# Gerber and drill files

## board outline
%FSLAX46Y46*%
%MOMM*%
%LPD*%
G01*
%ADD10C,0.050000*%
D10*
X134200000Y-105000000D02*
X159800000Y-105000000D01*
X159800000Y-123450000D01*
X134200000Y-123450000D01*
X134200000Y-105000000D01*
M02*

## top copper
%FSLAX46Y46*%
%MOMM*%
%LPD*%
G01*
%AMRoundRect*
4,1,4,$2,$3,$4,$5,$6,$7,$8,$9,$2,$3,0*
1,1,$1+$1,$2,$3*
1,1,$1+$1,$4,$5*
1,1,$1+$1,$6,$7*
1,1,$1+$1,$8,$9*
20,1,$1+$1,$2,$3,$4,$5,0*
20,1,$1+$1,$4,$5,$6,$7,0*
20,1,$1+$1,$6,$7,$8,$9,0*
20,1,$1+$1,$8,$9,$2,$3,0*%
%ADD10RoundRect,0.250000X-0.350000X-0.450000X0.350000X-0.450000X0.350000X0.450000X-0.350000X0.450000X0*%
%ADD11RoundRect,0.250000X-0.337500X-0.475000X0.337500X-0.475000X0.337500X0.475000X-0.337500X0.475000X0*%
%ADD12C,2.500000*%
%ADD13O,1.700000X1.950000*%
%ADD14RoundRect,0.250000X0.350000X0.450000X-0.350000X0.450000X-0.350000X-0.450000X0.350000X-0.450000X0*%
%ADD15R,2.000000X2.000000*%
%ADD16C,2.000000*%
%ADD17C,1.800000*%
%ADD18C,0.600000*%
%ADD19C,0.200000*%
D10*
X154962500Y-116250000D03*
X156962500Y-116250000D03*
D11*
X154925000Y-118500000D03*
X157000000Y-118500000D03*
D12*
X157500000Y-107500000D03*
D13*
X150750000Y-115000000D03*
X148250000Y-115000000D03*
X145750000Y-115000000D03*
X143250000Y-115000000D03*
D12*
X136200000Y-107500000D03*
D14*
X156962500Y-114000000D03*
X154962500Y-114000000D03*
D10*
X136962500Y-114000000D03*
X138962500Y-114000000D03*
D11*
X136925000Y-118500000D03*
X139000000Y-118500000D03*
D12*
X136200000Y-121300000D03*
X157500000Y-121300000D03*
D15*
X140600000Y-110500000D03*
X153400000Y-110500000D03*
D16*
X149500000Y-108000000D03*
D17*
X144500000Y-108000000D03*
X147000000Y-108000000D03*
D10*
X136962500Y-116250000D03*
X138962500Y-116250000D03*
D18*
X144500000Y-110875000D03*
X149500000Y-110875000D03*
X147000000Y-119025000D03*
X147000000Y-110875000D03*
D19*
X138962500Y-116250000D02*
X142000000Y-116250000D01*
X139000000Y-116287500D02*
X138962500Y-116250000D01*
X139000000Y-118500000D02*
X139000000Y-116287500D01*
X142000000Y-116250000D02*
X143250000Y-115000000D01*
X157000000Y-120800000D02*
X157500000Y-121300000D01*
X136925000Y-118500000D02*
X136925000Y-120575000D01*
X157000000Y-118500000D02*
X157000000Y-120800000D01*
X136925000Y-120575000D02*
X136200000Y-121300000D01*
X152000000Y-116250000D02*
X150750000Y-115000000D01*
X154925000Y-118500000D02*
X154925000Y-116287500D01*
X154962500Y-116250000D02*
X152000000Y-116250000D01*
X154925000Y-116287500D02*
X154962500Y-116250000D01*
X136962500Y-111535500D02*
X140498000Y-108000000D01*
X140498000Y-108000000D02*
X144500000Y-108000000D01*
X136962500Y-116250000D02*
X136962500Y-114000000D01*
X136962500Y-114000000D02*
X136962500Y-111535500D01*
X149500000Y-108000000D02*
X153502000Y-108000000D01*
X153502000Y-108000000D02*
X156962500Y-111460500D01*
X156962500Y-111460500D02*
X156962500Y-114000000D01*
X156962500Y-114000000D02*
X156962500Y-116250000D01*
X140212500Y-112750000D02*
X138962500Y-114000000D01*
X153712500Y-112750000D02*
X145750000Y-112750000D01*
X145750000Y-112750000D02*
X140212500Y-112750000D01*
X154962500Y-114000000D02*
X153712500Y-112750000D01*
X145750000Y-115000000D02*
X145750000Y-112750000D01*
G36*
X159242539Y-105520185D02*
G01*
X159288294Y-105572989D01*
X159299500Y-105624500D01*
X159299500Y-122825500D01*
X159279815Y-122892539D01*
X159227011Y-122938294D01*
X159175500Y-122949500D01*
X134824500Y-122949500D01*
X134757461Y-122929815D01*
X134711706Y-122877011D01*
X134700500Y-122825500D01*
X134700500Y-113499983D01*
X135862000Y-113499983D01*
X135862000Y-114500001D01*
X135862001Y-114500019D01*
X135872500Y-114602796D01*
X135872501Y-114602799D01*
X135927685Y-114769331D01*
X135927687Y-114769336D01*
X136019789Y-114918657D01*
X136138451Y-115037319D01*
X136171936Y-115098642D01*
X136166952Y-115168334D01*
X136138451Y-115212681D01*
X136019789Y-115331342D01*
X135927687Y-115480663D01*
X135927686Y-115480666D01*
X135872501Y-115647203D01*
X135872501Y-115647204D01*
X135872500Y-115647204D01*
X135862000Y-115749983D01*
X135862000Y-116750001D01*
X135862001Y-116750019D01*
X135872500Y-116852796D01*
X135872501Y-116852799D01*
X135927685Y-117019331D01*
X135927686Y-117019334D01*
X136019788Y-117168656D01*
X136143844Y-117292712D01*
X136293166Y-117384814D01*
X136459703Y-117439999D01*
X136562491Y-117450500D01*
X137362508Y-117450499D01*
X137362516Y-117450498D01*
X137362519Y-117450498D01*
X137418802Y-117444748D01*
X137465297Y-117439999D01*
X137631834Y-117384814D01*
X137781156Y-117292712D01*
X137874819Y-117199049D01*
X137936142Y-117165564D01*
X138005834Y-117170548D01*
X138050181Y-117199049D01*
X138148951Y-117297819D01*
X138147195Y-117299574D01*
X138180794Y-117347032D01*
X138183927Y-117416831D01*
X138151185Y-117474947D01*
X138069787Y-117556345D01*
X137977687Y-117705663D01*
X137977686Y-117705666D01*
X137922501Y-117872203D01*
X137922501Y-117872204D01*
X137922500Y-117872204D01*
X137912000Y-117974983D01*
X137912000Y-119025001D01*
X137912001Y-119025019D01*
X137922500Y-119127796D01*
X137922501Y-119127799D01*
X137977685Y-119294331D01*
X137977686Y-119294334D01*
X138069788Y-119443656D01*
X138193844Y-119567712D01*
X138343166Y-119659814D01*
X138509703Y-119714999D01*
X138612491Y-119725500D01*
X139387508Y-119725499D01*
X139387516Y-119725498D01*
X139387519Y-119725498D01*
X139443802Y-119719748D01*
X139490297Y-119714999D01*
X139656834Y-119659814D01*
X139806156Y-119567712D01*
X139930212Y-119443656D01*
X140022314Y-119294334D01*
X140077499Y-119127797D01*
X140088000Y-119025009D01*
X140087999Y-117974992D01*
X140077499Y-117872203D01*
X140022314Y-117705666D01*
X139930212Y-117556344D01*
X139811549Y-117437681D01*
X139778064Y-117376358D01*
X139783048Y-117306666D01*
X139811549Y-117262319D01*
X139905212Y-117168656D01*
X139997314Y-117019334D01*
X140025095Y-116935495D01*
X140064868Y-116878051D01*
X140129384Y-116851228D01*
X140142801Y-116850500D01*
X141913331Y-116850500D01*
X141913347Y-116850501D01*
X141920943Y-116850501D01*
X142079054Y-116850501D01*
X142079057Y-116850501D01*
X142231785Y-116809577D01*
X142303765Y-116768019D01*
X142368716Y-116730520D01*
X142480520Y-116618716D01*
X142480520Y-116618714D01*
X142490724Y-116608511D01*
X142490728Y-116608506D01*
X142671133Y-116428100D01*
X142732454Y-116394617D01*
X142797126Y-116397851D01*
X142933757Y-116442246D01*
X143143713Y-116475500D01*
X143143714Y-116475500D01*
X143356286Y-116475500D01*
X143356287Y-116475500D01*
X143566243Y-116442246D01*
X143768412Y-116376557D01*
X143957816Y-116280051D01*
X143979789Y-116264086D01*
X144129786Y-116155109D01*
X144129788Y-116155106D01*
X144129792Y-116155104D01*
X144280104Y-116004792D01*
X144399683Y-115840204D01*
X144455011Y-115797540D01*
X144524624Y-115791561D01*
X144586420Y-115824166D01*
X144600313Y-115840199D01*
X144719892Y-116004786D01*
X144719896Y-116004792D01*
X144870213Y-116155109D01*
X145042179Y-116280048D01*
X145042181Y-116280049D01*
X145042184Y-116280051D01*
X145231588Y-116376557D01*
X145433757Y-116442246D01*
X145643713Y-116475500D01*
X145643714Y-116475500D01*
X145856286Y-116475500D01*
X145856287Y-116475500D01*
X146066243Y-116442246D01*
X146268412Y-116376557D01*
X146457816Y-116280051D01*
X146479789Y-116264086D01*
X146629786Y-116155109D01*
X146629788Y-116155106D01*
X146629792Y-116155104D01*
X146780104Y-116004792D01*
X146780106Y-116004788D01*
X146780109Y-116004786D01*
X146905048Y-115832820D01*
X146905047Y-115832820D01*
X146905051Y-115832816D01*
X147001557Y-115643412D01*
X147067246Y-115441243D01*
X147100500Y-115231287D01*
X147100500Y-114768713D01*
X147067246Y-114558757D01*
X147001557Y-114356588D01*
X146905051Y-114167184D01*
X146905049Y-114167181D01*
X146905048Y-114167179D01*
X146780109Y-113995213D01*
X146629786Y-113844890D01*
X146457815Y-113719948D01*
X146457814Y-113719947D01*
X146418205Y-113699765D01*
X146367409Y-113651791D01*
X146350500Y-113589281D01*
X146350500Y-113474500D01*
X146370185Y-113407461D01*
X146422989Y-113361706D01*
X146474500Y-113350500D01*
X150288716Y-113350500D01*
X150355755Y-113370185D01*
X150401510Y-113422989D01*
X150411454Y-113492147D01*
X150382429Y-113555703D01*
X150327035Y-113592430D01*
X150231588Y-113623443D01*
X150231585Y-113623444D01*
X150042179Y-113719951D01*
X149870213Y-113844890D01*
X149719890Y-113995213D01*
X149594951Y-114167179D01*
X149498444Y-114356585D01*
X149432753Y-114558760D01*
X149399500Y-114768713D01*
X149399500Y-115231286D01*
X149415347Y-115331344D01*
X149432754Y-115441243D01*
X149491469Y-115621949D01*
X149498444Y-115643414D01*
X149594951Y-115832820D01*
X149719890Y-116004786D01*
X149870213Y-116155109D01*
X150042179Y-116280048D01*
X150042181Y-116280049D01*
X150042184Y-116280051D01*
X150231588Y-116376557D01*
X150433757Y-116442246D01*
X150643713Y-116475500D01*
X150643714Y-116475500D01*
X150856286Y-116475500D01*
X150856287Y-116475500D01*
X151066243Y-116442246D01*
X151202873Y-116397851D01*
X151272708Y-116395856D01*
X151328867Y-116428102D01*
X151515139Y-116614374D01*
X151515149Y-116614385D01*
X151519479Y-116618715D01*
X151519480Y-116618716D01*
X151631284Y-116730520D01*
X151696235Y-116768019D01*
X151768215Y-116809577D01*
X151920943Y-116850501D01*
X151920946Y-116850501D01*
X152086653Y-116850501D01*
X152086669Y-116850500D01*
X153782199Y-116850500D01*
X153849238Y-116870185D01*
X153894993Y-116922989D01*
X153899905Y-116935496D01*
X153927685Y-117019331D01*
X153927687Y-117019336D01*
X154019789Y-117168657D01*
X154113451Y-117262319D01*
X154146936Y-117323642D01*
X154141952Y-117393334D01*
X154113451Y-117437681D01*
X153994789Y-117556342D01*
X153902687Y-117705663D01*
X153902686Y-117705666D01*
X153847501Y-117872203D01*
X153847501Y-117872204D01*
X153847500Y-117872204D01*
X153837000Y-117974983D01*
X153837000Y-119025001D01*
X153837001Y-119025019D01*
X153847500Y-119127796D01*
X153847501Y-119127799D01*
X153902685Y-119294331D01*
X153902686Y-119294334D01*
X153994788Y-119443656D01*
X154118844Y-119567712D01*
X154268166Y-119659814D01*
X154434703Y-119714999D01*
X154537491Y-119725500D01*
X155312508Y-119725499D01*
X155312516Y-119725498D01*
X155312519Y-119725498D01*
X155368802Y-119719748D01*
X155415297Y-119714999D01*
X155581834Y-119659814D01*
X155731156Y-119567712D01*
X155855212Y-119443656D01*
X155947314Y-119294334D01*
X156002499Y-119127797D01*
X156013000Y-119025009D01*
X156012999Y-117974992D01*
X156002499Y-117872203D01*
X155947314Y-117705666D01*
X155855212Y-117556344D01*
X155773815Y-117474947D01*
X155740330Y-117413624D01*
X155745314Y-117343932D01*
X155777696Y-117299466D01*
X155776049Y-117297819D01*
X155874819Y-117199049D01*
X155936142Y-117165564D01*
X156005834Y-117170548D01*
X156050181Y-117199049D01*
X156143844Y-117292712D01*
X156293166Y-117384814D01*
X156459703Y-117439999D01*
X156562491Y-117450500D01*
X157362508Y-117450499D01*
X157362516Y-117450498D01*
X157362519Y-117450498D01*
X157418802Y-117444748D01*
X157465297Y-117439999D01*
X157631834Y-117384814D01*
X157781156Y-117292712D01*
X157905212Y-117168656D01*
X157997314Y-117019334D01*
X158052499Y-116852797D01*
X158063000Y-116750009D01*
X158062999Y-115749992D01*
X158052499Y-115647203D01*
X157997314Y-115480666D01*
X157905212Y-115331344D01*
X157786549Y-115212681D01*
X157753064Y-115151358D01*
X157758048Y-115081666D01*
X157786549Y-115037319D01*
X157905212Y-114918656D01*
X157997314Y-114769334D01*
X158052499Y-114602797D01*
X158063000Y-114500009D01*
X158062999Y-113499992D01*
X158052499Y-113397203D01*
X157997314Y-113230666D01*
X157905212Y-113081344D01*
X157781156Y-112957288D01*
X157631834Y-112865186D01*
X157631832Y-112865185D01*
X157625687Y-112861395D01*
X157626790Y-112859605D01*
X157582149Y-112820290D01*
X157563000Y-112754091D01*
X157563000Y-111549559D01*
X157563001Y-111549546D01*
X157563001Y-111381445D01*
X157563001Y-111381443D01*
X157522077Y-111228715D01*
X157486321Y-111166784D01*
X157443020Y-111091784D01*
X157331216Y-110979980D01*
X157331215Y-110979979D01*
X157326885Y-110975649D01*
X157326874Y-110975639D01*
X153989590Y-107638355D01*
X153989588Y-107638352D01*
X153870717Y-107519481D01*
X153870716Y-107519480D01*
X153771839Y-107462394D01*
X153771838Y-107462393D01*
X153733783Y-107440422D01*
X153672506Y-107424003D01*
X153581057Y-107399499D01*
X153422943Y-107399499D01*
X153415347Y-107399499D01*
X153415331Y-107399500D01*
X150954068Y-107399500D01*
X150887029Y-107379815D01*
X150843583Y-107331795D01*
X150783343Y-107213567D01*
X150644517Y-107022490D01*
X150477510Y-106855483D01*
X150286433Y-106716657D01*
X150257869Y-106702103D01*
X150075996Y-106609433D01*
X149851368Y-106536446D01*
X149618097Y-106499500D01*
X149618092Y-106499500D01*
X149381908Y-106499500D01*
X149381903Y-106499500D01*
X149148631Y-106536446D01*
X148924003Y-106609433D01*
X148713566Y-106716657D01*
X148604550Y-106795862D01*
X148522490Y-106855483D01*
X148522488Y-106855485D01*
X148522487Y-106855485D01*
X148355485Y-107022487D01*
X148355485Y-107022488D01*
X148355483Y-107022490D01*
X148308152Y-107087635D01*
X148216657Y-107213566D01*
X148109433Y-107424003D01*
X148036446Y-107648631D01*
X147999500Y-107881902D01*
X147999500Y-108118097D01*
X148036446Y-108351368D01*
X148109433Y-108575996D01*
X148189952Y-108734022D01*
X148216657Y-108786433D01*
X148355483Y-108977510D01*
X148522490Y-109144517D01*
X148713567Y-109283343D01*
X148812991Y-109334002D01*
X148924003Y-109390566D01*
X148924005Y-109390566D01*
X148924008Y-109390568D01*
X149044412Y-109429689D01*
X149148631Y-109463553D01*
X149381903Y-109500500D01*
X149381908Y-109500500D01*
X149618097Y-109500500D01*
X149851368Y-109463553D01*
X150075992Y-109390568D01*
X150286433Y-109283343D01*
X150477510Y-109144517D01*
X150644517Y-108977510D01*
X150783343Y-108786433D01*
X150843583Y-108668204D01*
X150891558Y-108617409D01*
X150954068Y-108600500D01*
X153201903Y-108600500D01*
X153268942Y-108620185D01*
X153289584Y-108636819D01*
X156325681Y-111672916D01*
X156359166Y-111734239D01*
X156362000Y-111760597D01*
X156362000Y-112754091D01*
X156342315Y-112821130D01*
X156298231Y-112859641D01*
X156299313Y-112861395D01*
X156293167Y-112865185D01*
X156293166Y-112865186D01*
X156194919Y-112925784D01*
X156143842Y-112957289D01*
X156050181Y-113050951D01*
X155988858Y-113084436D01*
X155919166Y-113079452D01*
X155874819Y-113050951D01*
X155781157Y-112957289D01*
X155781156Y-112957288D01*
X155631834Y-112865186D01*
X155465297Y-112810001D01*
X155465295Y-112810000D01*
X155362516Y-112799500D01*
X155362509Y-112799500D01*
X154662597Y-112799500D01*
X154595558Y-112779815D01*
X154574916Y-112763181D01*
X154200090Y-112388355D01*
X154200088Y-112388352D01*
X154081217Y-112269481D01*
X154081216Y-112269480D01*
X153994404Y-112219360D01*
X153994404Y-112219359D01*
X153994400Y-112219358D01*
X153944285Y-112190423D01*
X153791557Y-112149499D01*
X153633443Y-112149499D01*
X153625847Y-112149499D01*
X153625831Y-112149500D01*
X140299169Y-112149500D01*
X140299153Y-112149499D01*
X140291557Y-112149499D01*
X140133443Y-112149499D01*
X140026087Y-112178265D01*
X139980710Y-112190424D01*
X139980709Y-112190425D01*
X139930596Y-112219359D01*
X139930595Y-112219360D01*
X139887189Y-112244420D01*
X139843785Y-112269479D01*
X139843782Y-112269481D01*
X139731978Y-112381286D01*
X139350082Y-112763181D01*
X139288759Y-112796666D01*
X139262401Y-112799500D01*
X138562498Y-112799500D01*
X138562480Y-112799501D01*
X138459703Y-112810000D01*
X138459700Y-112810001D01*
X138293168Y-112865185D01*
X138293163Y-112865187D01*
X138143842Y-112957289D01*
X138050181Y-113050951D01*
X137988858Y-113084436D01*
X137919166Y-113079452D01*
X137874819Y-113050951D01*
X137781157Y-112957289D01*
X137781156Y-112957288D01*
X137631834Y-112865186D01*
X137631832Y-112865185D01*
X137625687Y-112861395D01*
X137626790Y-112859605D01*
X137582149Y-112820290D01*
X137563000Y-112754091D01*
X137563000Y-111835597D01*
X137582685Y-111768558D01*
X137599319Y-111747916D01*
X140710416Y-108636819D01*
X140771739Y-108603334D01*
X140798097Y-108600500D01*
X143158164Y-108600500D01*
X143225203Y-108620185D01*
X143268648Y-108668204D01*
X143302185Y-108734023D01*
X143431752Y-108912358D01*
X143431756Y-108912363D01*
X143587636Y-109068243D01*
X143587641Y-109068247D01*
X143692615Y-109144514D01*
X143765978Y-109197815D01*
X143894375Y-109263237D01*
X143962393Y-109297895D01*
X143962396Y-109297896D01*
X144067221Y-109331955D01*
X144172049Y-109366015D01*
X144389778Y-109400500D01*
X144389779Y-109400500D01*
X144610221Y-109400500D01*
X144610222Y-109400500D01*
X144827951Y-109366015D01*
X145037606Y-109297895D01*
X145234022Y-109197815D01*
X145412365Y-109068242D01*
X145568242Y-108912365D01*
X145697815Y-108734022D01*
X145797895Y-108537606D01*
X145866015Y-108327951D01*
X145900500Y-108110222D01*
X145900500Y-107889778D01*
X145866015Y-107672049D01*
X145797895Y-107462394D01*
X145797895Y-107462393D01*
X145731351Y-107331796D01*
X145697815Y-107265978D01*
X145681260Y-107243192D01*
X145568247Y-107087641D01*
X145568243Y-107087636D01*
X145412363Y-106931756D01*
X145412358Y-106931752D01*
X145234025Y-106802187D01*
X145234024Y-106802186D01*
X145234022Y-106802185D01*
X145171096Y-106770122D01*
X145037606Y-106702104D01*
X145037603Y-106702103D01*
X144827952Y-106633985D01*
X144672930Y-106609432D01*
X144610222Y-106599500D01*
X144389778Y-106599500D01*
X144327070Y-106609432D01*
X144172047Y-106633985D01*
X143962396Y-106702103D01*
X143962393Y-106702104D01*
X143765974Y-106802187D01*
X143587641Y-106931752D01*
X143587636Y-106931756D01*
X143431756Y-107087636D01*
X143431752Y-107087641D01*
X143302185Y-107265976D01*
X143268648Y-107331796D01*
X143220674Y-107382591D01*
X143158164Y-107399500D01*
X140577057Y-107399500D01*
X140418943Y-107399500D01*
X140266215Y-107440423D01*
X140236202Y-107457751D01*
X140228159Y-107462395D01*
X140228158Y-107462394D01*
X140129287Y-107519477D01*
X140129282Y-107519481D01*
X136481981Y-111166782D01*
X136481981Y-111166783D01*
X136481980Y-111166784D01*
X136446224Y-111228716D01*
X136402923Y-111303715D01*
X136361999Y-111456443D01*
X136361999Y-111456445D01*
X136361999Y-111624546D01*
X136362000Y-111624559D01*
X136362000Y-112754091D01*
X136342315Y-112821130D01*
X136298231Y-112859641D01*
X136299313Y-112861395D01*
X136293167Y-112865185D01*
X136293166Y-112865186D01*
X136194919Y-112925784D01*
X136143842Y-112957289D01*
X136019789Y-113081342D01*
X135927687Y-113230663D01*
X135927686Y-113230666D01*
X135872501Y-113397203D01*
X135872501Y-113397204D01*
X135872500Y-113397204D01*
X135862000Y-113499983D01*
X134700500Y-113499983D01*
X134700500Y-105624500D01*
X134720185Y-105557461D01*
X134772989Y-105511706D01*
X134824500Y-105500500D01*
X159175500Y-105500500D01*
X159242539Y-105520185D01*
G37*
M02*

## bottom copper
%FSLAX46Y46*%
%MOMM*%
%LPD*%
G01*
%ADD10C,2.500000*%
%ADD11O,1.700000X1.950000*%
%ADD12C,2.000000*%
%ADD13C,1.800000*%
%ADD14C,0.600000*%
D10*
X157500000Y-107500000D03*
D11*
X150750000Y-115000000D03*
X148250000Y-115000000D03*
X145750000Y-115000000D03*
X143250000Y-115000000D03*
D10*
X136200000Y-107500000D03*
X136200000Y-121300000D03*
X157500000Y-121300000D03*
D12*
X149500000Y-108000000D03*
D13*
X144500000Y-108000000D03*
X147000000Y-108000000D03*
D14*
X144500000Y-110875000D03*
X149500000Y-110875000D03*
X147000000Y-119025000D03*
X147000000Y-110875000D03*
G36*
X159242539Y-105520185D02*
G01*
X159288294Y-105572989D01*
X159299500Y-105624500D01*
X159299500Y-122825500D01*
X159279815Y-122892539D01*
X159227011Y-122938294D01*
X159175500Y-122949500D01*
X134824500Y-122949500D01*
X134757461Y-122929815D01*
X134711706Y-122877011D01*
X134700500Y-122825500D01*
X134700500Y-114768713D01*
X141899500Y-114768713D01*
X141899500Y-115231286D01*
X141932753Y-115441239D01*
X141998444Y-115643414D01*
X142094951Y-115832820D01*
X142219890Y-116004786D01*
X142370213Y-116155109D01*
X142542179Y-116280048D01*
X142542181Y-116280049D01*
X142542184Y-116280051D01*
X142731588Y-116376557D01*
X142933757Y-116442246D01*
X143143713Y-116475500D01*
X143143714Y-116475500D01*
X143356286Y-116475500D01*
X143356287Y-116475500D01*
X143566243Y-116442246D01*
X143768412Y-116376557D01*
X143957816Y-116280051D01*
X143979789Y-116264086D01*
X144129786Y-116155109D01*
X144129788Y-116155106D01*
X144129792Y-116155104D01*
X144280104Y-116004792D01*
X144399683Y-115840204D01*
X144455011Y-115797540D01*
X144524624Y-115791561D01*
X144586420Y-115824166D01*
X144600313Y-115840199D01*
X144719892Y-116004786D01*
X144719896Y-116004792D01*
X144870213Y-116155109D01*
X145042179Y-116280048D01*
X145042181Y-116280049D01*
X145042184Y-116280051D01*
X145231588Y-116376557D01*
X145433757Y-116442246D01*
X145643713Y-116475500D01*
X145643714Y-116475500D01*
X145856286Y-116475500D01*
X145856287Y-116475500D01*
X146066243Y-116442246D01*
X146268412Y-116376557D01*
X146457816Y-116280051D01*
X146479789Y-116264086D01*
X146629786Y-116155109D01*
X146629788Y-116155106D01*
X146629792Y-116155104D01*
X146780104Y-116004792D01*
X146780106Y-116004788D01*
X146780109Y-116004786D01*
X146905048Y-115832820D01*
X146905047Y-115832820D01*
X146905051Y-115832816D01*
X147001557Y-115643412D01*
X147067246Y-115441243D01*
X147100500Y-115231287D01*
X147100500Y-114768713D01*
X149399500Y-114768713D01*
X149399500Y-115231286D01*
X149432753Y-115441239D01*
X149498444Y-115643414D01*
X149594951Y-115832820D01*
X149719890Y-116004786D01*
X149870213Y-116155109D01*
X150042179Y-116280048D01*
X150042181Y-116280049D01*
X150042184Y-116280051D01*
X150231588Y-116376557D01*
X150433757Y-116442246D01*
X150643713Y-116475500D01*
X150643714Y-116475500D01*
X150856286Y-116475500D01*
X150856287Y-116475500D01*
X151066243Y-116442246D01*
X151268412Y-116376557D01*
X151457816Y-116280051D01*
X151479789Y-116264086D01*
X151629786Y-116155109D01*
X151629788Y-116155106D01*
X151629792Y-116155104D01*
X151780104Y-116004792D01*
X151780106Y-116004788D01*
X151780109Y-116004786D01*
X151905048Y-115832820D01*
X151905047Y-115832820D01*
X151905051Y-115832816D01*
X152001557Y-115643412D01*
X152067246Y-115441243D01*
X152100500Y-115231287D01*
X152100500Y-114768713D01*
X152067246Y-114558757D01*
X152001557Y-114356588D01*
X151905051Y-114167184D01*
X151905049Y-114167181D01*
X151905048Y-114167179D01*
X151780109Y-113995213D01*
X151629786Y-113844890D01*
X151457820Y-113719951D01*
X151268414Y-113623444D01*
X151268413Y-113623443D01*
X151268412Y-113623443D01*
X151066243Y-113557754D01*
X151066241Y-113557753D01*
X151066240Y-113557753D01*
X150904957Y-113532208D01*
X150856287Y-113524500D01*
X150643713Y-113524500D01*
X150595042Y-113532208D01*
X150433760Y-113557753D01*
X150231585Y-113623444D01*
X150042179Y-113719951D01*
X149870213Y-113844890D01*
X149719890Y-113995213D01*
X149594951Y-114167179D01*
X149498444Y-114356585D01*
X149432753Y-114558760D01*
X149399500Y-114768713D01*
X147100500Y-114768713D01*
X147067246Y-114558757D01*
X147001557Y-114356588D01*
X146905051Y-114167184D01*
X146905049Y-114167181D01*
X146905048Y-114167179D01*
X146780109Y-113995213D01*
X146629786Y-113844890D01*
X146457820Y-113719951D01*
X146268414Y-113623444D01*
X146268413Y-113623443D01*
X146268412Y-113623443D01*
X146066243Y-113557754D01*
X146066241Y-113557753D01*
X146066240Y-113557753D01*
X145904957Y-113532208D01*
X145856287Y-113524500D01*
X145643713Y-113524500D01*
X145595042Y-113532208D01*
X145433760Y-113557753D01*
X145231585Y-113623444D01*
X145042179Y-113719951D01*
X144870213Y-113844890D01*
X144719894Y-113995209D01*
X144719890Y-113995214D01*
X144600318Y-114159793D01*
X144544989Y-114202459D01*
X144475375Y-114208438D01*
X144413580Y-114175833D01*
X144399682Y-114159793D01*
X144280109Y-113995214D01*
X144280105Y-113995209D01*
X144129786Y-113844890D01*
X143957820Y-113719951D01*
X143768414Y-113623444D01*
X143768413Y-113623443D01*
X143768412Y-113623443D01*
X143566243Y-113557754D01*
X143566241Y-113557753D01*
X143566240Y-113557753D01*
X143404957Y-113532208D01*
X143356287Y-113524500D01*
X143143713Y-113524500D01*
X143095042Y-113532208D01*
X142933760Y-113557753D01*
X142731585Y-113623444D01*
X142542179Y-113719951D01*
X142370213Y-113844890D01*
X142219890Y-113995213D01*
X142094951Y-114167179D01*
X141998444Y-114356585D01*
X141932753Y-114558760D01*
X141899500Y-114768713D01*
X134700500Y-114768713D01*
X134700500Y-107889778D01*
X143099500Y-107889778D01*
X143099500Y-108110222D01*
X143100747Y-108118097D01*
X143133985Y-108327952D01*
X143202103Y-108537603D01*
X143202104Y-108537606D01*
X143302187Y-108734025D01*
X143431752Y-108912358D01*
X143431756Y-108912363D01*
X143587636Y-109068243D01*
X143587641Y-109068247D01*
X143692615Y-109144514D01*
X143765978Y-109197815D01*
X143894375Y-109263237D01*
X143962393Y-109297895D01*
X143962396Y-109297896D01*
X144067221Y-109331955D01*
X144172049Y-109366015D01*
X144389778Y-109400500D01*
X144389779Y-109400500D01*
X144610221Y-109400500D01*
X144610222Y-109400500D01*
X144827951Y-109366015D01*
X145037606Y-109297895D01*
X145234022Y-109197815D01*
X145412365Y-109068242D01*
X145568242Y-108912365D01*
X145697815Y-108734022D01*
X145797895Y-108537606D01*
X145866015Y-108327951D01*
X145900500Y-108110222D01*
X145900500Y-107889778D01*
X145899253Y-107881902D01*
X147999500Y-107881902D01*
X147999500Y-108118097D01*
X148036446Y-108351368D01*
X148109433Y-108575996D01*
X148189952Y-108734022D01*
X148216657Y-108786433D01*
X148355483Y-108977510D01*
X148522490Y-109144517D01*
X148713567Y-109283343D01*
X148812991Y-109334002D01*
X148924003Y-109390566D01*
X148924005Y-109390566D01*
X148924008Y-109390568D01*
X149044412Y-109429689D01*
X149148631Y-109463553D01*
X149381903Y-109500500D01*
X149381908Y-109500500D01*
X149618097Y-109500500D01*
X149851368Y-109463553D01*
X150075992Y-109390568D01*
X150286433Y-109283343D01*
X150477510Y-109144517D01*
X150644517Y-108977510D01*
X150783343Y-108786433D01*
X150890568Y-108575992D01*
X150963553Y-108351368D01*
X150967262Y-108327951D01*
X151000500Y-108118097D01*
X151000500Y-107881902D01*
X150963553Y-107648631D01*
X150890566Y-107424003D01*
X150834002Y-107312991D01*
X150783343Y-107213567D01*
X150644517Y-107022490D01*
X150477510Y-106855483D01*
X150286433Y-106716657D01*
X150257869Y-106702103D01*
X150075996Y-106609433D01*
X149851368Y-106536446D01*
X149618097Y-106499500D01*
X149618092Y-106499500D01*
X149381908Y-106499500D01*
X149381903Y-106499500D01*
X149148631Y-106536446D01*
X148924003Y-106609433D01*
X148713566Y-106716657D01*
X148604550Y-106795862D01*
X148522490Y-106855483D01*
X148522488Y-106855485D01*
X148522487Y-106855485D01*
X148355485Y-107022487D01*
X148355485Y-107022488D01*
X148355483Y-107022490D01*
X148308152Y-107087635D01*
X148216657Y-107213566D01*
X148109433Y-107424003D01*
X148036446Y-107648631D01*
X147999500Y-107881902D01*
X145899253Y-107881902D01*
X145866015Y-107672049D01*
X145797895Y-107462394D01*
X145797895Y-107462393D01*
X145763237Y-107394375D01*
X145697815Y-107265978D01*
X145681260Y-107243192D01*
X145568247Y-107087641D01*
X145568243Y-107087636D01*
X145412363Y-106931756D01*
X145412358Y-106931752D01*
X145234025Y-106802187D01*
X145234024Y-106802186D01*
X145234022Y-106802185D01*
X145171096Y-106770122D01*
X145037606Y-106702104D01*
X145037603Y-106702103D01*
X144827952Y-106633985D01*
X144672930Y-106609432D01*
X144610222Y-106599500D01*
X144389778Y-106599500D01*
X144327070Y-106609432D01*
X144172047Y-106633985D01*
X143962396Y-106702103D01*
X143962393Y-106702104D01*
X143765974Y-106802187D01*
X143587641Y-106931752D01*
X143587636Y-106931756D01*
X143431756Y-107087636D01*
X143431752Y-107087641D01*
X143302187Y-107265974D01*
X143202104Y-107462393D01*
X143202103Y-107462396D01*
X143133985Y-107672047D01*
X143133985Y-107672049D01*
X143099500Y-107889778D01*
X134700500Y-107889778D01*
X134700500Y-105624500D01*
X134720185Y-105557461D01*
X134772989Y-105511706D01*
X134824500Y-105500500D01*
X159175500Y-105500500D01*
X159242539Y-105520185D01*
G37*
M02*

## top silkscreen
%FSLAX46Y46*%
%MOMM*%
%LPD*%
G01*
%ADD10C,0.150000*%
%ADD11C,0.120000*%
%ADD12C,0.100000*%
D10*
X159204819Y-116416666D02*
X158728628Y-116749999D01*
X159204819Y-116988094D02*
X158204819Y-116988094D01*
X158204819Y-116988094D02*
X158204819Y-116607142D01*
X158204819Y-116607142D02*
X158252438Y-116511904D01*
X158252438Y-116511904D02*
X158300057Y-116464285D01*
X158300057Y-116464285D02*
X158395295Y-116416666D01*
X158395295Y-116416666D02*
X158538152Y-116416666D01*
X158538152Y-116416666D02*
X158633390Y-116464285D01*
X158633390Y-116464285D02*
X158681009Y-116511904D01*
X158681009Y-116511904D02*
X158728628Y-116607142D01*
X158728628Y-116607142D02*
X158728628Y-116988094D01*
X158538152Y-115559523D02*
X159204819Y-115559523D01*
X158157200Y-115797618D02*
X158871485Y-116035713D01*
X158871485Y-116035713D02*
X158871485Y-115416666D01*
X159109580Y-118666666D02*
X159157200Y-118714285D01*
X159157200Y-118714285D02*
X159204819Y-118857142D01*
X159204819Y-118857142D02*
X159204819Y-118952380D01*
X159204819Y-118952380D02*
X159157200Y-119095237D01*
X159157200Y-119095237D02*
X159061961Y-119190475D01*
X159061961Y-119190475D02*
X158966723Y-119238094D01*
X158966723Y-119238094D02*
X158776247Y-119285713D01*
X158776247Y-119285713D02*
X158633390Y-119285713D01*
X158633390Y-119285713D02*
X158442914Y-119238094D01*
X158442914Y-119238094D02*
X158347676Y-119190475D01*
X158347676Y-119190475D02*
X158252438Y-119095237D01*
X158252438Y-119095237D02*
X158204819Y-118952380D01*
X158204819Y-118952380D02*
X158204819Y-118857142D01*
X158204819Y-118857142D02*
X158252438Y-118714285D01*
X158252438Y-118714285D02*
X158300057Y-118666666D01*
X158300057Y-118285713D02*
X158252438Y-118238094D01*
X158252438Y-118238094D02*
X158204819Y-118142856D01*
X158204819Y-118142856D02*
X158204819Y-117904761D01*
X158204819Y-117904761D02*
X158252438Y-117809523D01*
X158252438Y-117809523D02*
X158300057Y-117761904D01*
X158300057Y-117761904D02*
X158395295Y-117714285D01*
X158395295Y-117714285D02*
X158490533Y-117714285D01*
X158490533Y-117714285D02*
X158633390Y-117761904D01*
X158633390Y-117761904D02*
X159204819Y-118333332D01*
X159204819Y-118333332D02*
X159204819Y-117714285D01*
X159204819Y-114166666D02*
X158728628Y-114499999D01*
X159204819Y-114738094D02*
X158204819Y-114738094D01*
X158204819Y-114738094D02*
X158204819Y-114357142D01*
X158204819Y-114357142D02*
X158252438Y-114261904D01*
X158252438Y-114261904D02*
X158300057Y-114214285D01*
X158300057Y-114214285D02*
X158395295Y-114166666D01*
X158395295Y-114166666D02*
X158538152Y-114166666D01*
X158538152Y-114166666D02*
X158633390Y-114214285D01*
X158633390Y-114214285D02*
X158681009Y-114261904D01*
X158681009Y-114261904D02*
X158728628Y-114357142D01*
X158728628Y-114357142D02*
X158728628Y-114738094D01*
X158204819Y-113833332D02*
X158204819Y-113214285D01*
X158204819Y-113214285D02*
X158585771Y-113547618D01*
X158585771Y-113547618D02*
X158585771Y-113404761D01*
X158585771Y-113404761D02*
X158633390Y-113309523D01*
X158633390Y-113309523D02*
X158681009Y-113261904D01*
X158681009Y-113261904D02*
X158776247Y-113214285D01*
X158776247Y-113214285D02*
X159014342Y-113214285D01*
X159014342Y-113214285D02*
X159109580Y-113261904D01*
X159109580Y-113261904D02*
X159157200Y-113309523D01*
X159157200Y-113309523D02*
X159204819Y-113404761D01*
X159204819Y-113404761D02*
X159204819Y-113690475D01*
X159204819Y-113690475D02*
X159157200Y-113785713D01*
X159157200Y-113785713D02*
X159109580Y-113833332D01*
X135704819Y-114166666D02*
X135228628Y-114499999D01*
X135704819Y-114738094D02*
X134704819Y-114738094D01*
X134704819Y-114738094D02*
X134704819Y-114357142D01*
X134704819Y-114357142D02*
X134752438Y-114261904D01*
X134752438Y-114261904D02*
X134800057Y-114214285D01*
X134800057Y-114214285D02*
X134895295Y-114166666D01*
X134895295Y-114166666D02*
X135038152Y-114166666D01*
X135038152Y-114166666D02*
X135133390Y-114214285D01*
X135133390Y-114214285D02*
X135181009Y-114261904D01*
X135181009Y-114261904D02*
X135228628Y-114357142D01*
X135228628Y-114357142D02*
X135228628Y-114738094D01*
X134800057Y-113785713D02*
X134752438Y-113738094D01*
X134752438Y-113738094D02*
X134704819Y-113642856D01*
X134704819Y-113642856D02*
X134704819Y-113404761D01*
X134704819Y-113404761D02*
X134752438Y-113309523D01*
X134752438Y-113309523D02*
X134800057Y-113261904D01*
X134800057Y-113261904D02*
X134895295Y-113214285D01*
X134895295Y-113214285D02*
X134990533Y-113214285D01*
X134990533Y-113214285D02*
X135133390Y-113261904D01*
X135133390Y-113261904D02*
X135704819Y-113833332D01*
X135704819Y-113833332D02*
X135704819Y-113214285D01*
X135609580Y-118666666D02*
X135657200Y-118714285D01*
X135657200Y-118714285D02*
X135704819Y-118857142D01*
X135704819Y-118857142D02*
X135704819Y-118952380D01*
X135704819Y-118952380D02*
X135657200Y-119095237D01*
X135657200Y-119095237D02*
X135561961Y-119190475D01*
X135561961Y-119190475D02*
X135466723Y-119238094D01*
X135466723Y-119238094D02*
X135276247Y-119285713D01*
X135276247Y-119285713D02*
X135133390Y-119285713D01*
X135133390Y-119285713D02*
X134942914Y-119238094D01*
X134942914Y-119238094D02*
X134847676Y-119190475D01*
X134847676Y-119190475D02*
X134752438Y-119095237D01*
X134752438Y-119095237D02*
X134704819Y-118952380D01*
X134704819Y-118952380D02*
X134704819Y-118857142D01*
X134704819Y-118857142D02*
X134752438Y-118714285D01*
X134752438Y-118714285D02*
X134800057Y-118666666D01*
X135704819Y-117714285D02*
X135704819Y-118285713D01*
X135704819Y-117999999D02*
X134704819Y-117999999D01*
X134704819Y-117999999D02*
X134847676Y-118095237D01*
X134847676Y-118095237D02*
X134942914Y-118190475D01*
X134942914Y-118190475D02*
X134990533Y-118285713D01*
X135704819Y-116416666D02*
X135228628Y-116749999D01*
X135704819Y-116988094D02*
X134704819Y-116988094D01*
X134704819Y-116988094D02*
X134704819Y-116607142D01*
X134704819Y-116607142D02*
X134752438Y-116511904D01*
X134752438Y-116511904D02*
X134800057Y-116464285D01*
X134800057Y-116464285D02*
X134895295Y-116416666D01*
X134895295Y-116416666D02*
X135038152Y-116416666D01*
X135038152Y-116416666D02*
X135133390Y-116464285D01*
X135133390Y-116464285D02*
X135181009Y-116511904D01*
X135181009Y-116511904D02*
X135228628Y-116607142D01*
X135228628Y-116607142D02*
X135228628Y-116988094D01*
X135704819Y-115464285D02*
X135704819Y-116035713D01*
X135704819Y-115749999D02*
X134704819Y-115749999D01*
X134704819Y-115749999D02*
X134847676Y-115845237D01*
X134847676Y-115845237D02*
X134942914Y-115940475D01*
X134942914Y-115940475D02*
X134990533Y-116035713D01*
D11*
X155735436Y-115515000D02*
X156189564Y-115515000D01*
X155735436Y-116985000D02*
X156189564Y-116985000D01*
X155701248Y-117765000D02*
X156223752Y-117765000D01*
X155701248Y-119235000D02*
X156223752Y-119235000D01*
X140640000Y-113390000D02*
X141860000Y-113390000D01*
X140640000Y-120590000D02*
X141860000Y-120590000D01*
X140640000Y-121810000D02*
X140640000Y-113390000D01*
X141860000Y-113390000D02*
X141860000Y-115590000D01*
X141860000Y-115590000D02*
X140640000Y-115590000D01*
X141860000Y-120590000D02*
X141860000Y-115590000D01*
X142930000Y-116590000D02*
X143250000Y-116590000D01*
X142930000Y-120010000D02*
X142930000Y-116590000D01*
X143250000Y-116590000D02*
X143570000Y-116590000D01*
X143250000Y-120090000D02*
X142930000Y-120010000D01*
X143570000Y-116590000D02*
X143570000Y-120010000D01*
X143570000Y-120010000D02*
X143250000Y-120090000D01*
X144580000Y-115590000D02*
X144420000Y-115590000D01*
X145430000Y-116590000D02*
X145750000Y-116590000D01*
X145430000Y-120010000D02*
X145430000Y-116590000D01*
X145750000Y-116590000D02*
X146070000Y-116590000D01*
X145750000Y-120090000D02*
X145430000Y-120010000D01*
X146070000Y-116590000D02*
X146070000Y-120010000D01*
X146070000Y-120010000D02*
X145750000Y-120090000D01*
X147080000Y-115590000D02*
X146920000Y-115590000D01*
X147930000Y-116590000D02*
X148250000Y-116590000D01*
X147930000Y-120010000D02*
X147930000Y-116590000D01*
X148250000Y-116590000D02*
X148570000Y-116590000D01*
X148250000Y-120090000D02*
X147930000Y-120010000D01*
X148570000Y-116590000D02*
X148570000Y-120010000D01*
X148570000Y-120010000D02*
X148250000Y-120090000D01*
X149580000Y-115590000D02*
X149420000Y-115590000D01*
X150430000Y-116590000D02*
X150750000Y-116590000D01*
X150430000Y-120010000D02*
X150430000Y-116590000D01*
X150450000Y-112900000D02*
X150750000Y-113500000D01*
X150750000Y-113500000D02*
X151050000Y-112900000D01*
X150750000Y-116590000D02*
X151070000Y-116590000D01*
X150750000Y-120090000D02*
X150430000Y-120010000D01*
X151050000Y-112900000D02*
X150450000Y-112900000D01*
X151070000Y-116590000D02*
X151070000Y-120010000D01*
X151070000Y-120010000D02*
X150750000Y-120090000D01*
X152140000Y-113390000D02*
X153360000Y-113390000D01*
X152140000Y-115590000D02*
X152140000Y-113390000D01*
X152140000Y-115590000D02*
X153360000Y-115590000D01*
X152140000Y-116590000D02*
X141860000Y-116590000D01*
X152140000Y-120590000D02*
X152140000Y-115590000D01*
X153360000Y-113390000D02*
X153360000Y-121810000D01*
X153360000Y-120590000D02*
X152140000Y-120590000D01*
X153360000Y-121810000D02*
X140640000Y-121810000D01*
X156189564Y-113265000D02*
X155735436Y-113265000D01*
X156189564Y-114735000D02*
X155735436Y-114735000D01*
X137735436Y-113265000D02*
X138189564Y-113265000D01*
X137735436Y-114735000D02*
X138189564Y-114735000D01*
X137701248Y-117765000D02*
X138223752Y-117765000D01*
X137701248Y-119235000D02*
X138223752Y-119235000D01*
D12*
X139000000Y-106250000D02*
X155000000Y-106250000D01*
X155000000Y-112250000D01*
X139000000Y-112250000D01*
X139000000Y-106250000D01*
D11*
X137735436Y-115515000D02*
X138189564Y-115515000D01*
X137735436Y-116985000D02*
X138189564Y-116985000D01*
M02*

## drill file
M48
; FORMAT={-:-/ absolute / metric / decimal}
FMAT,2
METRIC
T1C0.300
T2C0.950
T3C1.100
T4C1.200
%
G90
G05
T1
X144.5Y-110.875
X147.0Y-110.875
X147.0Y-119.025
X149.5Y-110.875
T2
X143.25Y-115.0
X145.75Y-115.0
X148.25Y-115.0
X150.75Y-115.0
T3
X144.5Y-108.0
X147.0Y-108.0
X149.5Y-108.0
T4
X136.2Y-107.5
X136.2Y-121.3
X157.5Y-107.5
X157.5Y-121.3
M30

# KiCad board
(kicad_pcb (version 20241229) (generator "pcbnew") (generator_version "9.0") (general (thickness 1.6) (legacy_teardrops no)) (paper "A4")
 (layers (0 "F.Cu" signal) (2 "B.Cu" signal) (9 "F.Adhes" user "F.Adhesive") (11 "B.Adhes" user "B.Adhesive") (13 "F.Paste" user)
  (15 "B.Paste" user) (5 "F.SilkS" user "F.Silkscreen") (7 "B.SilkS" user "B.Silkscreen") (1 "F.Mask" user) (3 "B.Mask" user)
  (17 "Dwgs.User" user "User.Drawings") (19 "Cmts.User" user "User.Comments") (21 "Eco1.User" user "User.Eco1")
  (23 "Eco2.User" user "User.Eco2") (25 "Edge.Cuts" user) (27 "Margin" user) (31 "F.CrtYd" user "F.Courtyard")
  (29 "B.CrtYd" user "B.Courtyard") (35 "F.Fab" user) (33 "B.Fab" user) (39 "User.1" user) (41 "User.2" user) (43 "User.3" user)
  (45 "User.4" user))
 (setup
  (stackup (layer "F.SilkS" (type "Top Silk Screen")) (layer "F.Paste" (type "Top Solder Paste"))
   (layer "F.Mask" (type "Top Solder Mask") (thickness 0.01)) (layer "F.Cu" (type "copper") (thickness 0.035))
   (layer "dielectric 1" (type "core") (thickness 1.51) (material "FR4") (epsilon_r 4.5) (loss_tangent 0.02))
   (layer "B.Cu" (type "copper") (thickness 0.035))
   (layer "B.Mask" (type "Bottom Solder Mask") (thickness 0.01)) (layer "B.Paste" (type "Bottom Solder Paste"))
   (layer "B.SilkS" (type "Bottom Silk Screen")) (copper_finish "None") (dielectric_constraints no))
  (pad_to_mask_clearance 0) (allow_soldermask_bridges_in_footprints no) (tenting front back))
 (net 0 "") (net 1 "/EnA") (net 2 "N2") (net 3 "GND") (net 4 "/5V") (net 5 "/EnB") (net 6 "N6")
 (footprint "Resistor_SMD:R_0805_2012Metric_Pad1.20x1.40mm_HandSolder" (layer "F.Cu") (at 155.9625 116.25)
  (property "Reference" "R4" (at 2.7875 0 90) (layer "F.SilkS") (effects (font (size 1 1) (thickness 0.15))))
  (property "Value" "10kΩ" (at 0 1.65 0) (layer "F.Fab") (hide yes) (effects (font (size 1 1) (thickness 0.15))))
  (fp_line (start -0.227064 -0.735) (end 0.227064 -0.735) (stroke (width 0.12) (type solid)) (layer "F.SilkS"))
  (fp_line (start -0.227064 0.735) (end 0.227064 0.735) (stroke (width 0.12) (type solid)) (layer "F.SilkS"))
  (pad "1" smd roundrect (at -1 0) (size 1.2 1.4) (layers "F.Cu" "F.Mask" "F.Paste") (roundrect_rratio 0.208333) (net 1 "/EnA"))
  (pad "2" smd roundrect (at 1 0) (size 1.2 1.4) (layers "F.Cu" "F.Mask" "F.Paste") (roundrect_rratio 0.208333) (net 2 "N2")))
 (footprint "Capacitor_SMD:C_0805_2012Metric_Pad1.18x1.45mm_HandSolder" (layer "F.Cu") (at 155.9625 118.5)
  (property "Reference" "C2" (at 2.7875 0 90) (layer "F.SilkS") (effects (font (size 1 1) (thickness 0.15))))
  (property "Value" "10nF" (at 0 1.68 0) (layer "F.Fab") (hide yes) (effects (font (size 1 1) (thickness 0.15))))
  (fp_line (start -0.261252 -0.735) (end 0.261252 -0.735) (stroke (width 0.12) (type solid)) (layer "F.SilkS"))
  (fp_line (start -0.261252 0.735) (end 0.261252 0.735) (stroke (width 0.12) (type solid)) (layer "F.SilkS"))
  (pad "1" smd roundrect (at -1.0375 0) (size 1.175 1.45) (layers "F.Cu" "F.Mask" "F.Paste") (roundrect_rratio 0.212766) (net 1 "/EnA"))
  (pad "2" smd roundrect (at 1.0375 0) (size 1.175 1.45) (layers "F.Cu" "F.Mask" "F.Paste") (roundrect_rratio 0.212766) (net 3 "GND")))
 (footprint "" (layer "F.Cu") (at 157.5 107.5)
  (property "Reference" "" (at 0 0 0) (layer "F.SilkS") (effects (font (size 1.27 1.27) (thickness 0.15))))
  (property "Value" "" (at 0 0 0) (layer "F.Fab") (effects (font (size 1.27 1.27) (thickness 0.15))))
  (pad "" thru_hole circle (at 0 0 90) (size 2.5 2.5) (drill 1.2) (layers "*.Cu" "*.Mask") (remove_unused_layers no) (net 3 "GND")))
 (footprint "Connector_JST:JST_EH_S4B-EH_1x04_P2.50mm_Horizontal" (layer "F.Cu") (at 150.75 115 180)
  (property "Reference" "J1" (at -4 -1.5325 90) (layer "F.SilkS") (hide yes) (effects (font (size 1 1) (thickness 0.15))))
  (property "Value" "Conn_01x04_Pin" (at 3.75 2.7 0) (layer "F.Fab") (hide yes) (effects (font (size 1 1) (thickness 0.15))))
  (fp_line (start 10.11 1.61) (end 8.89 1.61) (stroke (width 0.12) (type solid)) (layer "F.SilkS"))
  (fp_line (start 10.11 -5.59) (end 8.89 -5.59) (stroke (width 0.12) (type solid)) (layer "F.SilkS"))
  (fp_line (start 10.11 -6.81) (end 10.11 1.61) (stroke (width 0.12) (type solid)) (layer "F.SilkS"))
  (fp_line (start 8.89 1.61) (end 8.89 -0.59) (stroke (width 0.12) (type solid)) (layer "F.SilkS"))
  (fp_line (start 8.89 -0.59) (end 10.11 -0.59) (stroke (width 0.12) (type solid)) (layer "F.SilkS"))
  (fp_line (start 8.89 -5.59) (end 8.89 -0.59) (stroke (width 0.12) (type solid)) (layer "F.SilkS"))
  (fp_line (start 7.82 -1.59) (end 7.5 -1.59) (stroke (width 0.12) (type solid)) (layer "F.SilkS"))
  (fp_line (start 7.82 -5.01) (end 7.82 -1.59) (stroke (width 0.12) (type solid)) (layer "F.SilkS"))
  (fp_line (start 7.5 -1.59) (end 7.18 -1.59) (stroke (width 0.12) (type solid)) (layer "F.SilkS"))
  (fp_line (start 7.5 -5.09) (end 7.82 -5.01) (stroke (width 0.12) (type solid)) (layer "F.SilkS"))
  (fp_line (start 7.18 -1.59) (end 7.18 -5.01) (stroke (width 0.12) (type solid)) (layer "F.SilkS"))
  (fp_line (start 7.18 -5.01) (end 7.5 -5.09) (stroke (width 0.12) (type solid)) (layer "F.SilkS"))
  (fp_line (start 6.17 -0.59) (end 6.33 -0.59) (stroke (width 0.12) (type solid)) (layer "F.SilkS"))
  (fp_line (start 5.32 -1.59) (end 5 -1.59) (stroke (width 0.12) (type solid)) (layer "F.SilkS"))
  (fp_line (start 5.32 -5.01) (end 5.32 -1.59) (stroke (width 0.12) (type solid)) (layer "F.SilkS"))
  (fp_line (start 5 -1.59) (end 4.68 -1.59) (stroke (width 0.12) (type solid)) (layer "F.SilkS"))
  (fp_line (start 5 -5.09) (end 5.32 -5.01) (stroke (width 0.12) (type solid)) (layer "F.SilkS"))
  (fp_line (start 4.68 -1.59) (end 4.68 -5.01) (stroke (width 0.12) (type solid)) (layer "F.SilkS"))
  (fp_line (start 4.68 -5.01) (end 5 -5.09) (stroke (width 0.12) (type solid)) (layer "F.SilkS"))
  (fp_line (start 3.67 -0.59) (end 3.83 -0.59) (stroke (width 0.12) (type solid)) (layer "F.SilkS"))
  (fp_line (start 2.82 -1.59) (end 2.5 -1.59) (stroke (width 0.12) (type solid)) (layer "F.SilkS"))
  (fp_line (start 2.82 -5.01) (end 2.82 -1.59) (stroke (width 0.12) (type solid)) (layer "F.SilkS"))
  (fp_line (start 2.5 -1.59) (end 2.18 -1.59) (stroke (width 0.12) (type solid)) (layer "F.SilkS"))
  (fp_line (start 2.5 -5.09) (end 2.82 -5.01) (stroke (width 0.12) (type solid)) (layer "F.SilkS"))
  (fp_line (start 2.18 -1.59) (end 2.18 -5.01) (stroke (width 0.12) (type solid)) (layer "F.SilkS"))
  (fp_line (start 2.18 -5.01) (end 2.5 -5.09) (stroke (width 0.12) (type solid)) (layer "F.SilkS"))
  (fp_line (start 1.17 -0.59) (end 1.33 -0.59) (stroke (width 0.12) (type solid)) (layer "F.SilkS"))
  (fp_line (start 0.32 -1.59) (end 0 -1.59) (stroke (width 0.12) (type solid)) (layer "F.SilkS"))
  (fp_line (start 0.32 -5.01) (end 0.32 -1.59) (stroke (width 0.12) (type solid)) (layer "F.SilkS"))
  (fp_line (start 0.3 2.1) (end 0 1.5) (stroke (width 0.12) (type solid)) (layer "F.SilkS"))
  (fp_line (start 0 1.5) (end -0.3 2.1) (stroke (width 0.12) (type solid)) (layer "F.SilkS"))
  (fp_line (start 0 -1.59) (end -0.32 -1.59) (stroke (width 0.12) (type solid)) (layer "F.SilkS"))
  (fp_line (start 0 -5.09) (end 0.32 -5.01) (stroke (width 0.12) (type solid)) (layer "F.SilkS"))
  (fp_line (start -0.3 2.1) (end 0.3 2.1) (stroke (width 0.12) (type solid)) (layer "F.SilkS"))
  (fp_line (start -0.32 -1.59) (end -0.32 -5.01) (stroke (width 0.12) (type solid)) (layer "F.SilkS"))
  (fp_line (start -0.32 -5.01) (end 0 -5.09) (stroke (width 0.12) (type solid)) (layer "F.SilkS"))
  (fp_line (start -1.39 1.61) (end -2.61 1.61) (stroke (width 0.12) (type solid)) (layer "F.SilkS"))
  (fp_line (start -1.39 -0.59) (end -1.39 1.61) (stroke (width 0.12) (type solid)) (layer "F.SilkS"))
  (fp_line (start -1.39 -0.59) (end -2.61 -0.59) (stroke (width 0.12) (type solid)) (layer "F.SilkS"))
  (fp_line (start -1.39 -1.59) (end 8.89 -1.59) (stroke (width 0.12) (type solid)) (layer "F.SilkS"))
  (fp_line (start -1.39 -5.59) (end -1.39 -0.59) (stroke (width 0.12) (type solid)) (layer "F.SilkS"))
  (fp_line (start -2.61 1.61) (end -2.61 -6.81) (stroke (width 0.12) (type solid)) (layer "F.SilkS"))
  (fp_line (start -2.61 -5.59) (end -1.39 -5.59) (stroke (width 0.12) (type solid)) (layer "F.SilkS"))
  (fp_line (start -2.61 -6.81) (end 10.11 -6.81) (stroke (width 0.12) (type solid)) (layer "F.SilkS"))
  (pad "1" thru_hole oval (at 0 0 180) (size 1.7 1.95) (drill 0.95) (layers "*.Cu" "*.Mask") (remove_unused_layers no) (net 1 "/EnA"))
  (pad "2" thru_hole oval (at 2.5 0 180) (size 1.7 1.95) (drill 0.95) (layers "*.Cu" "*.Mask") (remove_unused_layers no) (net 3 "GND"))
  (pad "3" thru_hole oval (at 5 0 180) (size 1.7 1.95) (drill 0.95) (layers "*.Cu" "*.Mask") (remove_unused_layers no) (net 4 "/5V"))
  (pad "4" thru_hole oval (at 7.5 0 180) (size 1.7 1.95) (drill 0.95) (layers "*.Cu" "*.Mask") (remove_unused_layers no) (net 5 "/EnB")))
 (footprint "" (layer "F.Cu") (at 136.2 107.5)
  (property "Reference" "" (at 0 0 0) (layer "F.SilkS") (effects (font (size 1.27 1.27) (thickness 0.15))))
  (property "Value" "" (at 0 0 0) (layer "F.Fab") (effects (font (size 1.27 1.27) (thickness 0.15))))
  (pad "" thru_hole circle (at 0 0 90) (size 2.5 2.5) (drill 1.2) (layers "*.Cu" "*.Mask") (remove_unused_layers no) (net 3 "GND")))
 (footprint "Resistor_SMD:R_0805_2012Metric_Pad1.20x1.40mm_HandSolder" (layer "F.Cu") (at 155.9625 114 180)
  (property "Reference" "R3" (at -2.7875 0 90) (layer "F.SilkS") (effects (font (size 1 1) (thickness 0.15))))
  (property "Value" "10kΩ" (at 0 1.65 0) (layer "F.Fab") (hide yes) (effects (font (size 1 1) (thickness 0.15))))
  (fp_line (start -0.227064 0.735) (end 0.227064 0.735) (stroke (width 0.12) (type solid)) (layer "F.SilkS"))
  (fp_line (start -0.227064 -0.735) (end 0.227064 -0.735) (stroke (width 0.12) (type solid)) (layer "F.SilkS"))
  (pad "1" smd roundrect (at -1 0 180) (size 1.2 1.4) (layers "F.Cu" "F.Mask" "F.Paste") (roundrect_rratio 0.208333) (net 2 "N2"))
  (pad "2" smd roundrect (at 1 0 180) (size 1.2 1.4) (layers "F.Cu" "F.Mask" "F.Paste") (roundrect_rratio 0.208333) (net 4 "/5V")))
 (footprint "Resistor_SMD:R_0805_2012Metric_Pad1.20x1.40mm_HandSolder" (layer "F.Cu") (at 137.9625 114)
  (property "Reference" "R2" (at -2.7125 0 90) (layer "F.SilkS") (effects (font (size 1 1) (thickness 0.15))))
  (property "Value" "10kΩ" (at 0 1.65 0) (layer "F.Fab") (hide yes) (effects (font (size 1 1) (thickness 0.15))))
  (fp_line (start -0.227064 -0.735) (end 0.227064 -0.735) (stroke (width 0.12) (type solid)) (layer "F.SilkS"))
  (fp_line (start -0.227064 0.735) (end 0.227064 0.735) (stroke (width 0.12) (type solid)) (layer "F.SilkS"))
  (pad "1" smd roundrect (at -1 0) (size 1.2 1.4) (layers "F.Cu" "F.Mask" "F.Paste") (roundrect_rratio 0.208333) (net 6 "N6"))
  (pad "2" smd roundrect (at 1 0) (size 1.2 1.4) (layers "F.Cu" "F.Mask" "F.Paste") (roundrect_rratio 0.208333) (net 4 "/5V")))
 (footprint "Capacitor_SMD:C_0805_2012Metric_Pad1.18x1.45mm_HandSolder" (layer "F.Cu") (at 137.9625 118.5)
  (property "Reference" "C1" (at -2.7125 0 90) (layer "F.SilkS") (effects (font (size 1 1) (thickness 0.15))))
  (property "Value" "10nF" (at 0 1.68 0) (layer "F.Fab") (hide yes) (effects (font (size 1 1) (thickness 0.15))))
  (fp_line (start -0.261252 -0.735) (end 0.261252 -0.735) (stroke (width 0.12) (type solid)) (layer "F.SilkS"))
  (fp_line (start -0.261252 0.735) (end 0.261252 0.735) (stroke (width 0.12) (type solid)) (layer "F.SilkS"))
  (pad "1" smd roundrect (at -1.0375 0) (size 1.175 1.45) (layers "F.Cu" "F.Mask" "F.Paste") (roundrect_rratio 0.212766) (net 3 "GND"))
  (pad "2" smd roundrect (at 1.0375 0) (size 1.175 1.45) (layers "F.Cu" "F.Mask" "F.Paste") (roundrect_rratio 0.212766) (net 5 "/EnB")))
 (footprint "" (layer "F.Cu") (at 136.2 121.3 90)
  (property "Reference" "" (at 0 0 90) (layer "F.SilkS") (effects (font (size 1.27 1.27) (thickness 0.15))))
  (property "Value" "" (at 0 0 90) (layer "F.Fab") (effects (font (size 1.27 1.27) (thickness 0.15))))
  (pad "" thru_hole circle (at 0 0 180) (size 2.5 2.5) (drill 1.2) (layers "*.Cu" "*.Mask") (remove_unused_layers no) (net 3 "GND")))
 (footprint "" (layer "F.Cu") (at 157.5 121.3)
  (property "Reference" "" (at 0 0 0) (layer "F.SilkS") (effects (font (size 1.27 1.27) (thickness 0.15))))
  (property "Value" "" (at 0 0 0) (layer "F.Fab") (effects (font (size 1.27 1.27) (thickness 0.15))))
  (pad "" thru_hole circle (at 0 0 90) (size 2.5 2.5) (drill 1.2) (layers "*.Cu" "*.Mask") (remove_unused_layers no) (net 3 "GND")))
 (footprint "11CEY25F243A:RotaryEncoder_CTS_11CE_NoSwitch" (layer "F.Cu") (at 149.5 108 90)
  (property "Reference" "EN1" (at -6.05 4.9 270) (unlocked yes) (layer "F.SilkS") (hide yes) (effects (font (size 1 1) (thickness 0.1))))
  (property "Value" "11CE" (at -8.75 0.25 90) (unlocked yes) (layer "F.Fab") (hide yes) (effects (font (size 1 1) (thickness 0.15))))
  (fp_rect (start -4.25 -10.5) (end 1.75 5.5) (stroke (width 0.1) (type default)) (fill no) (layer "F.SilkS"))
  (pad "1" smd rect (at -2.5 -8.9 90) (size 2 2) (layers "F.Cu" "F.Mask" "F.Paste") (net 3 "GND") (thermal_bridge_angle 45))
  (pad "2" smd rect (at -2.5 3.9 90) (size 2 2) (layers "F.Cu" "F.Mask" "F.Paste") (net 3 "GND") (thermal_bridge_angle 45))
  (pad "A" thru_hole circle (at 0 0 90) (size 2 2) (drill 1.1) (layers "*.Cu" "*.Mask") (remove_unused_layers no) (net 2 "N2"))
  (pad "B" thru_hole circle (at 0 -5 90) (size 1.8 1.8) (drill 1.1) (layers "*.Cu" "*.Mask") (remove_unused_layers no) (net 6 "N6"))
  (pad "C" thru_hole circle (at 0 -2.5 90) (size 1.8 1.8) (drill 1.1) (layers "*.Cu" "*.Mask") (remove_unused_layers no) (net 3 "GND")))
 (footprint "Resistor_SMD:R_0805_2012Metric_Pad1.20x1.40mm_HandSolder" (layer "F.Cu") (at 137.9625 116.25)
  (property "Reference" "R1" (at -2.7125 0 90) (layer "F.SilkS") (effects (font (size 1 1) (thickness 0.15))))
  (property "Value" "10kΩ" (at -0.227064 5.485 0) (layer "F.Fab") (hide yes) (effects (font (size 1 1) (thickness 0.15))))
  (fp_line (start -0.227064 -0.735) (end 0.227064 -0.735) (stroke (width 0.12) (type solid)) (layer "F.SilkS"))
  (fp_line (start -0.227064 0.735) (end 0.227064 0.735) (stroke (width 0.12) (type solid)) (layer "F.SilkS"))
  (pad "1" smd roundrect (at -1 0) (size 1.2 1.4) (layers "F.Cu" "F.Mask" "F.Paste") (roundrect_rratio 0.208333) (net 6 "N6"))
  (pad "2" smd roundrect (at 1 0) (size 1.2 1.4) (layers "F.Cu" "F.Mask" "F.Paste") (roundrect_rratio 0.208333) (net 5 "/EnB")))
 (gr_rect (start 134.2 105) (end 159.8 123.45) (stroke (width 0.05) (type default)) (fill no) (layer "Edge.Cuts"))
 (segment (start 138.9625 116.25) (end 142 116.25) (width 0.2) (layer "F.Cu") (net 5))
 (segment (start 139 116.2875) (end 138.9625 116.25) (width 0.2) (layer "F.Cu") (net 5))
 (segment (start 139 118.5) (end 139 116.2875) (width 0.2) (layer "F.Cu") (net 5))
 (segment (start 142 116.25) (end 143.25 115) (width 0.2) (layer "F.Cu") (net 5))
 (segment (start 157 120.8) (end 157.5 121.3) (width 0.2) (layer "F.Cu") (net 3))
 (segment (start 136.925 118.5) (end 136.925 120.575) (width 0.2) (layer "F.Cu") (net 3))
 (segment (start 157 118.5) (end 157 120.8) (width 0.2) (layer "F.Cu") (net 3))
 (segment (start 136.925 120.575) (end 136.2 121.3) (width 0.2) (layer "F.Cu") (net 3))
 (via (at 144.5 110.875) (size 0.6) (drill 0.3) (layers "F.Cu" "B.Cu") (free yes) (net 3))
 (via (at 149.5 110.875) (size 0.6) (drill 0.3) (layers "F.Cu" "B.Cu") (free yes) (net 3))
 (via (at 147 119.025) (size 0.6) (drill 0.3) (layers "F.Cu" "B.Cu") (free yes) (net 3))
 (via (at 147 110.875) (size 0.6) (drill 0.3) (layers "F.Cu" "B.Cu") (free yes) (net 3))
 (segment (start 152 116.25) (end 150.75 115) (width 0.2) (layer "F.Cu") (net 1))
 (segment (start 154.925 118.5) (end 154.925 116.2875) (width 0.2) (layer "F.Cu") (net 1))
 (segment (start 154.9625 116.25) (end 152 116.25) (width 0.2) (layer "F.Cu") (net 1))
 (segment (start 154.925 116.2875) (end 154.9625 116.25) (width 0.2) (layer "F.Cu") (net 1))
 (segment (start 136.9625 111.5355) (end 140.498 108) (width 0.2) (layer "F.Cu") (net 6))
 (segment (start 140.498 108) (end 144.5 108) (width 0.2) (layer "F.Cu") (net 6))
 (segment (start 136.9625 116.25) (end 136.9625 114) (width 0.2) (layer "F.Cu") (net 6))
 (segment (start 136.9625 114) (end 136.9625 111.5355) (width 0.2) (layer "F.Cu") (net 6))
 (segment (start 149.5 108) (end 153.502 108) (width 0.2) (layer "F.Cu") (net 2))
 (segment (start 153.502 108) (end 156.9625 111.4605) (width 0.2) (layer "F.Cu") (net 2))
 (segment (start 156.9625 111.4605) (end 156.9625 114) (width 0.2) (layer "F.Cu") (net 2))
 (segment (start 156.9625 114) (end 156.9625 116.25) (width 0.2) (layer "F.Cu") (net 2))
 (segment (start 140.2125 112.75) (end 138.9625 114) (width 0.2) (layer "F.Cu") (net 4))
 (segment (start 153.7125 112.75) (end 145.75 112.75) (width 0.2) (layer "F.Cu") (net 4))
 (segment (start 145.75 112.75) (end 140.2125 112.75) (width 0.2) (layer "F.Cu") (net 4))
 (segment (start 154.9625 114) (end 153.7125 112.75) (width 0.2) (layer "F.Cu") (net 4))
 (segment (start 145.75 115) (end 145.75 112.75) (width 0.2) (layer "F.Cu") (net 4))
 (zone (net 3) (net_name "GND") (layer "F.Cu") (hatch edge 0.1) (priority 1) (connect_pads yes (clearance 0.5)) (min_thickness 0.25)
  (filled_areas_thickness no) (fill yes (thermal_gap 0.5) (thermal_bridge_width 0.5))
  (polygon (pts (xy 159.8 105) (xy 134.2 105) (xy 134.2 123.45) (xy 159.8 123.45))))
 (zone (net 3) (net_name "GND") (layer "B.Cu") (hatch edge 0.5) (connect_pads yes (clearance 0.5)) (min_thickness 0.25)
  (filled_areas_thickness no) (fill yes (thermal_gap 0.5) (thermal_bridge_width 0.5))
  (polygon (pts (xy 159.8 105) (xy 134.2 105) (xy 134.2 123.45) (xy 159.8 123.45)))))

